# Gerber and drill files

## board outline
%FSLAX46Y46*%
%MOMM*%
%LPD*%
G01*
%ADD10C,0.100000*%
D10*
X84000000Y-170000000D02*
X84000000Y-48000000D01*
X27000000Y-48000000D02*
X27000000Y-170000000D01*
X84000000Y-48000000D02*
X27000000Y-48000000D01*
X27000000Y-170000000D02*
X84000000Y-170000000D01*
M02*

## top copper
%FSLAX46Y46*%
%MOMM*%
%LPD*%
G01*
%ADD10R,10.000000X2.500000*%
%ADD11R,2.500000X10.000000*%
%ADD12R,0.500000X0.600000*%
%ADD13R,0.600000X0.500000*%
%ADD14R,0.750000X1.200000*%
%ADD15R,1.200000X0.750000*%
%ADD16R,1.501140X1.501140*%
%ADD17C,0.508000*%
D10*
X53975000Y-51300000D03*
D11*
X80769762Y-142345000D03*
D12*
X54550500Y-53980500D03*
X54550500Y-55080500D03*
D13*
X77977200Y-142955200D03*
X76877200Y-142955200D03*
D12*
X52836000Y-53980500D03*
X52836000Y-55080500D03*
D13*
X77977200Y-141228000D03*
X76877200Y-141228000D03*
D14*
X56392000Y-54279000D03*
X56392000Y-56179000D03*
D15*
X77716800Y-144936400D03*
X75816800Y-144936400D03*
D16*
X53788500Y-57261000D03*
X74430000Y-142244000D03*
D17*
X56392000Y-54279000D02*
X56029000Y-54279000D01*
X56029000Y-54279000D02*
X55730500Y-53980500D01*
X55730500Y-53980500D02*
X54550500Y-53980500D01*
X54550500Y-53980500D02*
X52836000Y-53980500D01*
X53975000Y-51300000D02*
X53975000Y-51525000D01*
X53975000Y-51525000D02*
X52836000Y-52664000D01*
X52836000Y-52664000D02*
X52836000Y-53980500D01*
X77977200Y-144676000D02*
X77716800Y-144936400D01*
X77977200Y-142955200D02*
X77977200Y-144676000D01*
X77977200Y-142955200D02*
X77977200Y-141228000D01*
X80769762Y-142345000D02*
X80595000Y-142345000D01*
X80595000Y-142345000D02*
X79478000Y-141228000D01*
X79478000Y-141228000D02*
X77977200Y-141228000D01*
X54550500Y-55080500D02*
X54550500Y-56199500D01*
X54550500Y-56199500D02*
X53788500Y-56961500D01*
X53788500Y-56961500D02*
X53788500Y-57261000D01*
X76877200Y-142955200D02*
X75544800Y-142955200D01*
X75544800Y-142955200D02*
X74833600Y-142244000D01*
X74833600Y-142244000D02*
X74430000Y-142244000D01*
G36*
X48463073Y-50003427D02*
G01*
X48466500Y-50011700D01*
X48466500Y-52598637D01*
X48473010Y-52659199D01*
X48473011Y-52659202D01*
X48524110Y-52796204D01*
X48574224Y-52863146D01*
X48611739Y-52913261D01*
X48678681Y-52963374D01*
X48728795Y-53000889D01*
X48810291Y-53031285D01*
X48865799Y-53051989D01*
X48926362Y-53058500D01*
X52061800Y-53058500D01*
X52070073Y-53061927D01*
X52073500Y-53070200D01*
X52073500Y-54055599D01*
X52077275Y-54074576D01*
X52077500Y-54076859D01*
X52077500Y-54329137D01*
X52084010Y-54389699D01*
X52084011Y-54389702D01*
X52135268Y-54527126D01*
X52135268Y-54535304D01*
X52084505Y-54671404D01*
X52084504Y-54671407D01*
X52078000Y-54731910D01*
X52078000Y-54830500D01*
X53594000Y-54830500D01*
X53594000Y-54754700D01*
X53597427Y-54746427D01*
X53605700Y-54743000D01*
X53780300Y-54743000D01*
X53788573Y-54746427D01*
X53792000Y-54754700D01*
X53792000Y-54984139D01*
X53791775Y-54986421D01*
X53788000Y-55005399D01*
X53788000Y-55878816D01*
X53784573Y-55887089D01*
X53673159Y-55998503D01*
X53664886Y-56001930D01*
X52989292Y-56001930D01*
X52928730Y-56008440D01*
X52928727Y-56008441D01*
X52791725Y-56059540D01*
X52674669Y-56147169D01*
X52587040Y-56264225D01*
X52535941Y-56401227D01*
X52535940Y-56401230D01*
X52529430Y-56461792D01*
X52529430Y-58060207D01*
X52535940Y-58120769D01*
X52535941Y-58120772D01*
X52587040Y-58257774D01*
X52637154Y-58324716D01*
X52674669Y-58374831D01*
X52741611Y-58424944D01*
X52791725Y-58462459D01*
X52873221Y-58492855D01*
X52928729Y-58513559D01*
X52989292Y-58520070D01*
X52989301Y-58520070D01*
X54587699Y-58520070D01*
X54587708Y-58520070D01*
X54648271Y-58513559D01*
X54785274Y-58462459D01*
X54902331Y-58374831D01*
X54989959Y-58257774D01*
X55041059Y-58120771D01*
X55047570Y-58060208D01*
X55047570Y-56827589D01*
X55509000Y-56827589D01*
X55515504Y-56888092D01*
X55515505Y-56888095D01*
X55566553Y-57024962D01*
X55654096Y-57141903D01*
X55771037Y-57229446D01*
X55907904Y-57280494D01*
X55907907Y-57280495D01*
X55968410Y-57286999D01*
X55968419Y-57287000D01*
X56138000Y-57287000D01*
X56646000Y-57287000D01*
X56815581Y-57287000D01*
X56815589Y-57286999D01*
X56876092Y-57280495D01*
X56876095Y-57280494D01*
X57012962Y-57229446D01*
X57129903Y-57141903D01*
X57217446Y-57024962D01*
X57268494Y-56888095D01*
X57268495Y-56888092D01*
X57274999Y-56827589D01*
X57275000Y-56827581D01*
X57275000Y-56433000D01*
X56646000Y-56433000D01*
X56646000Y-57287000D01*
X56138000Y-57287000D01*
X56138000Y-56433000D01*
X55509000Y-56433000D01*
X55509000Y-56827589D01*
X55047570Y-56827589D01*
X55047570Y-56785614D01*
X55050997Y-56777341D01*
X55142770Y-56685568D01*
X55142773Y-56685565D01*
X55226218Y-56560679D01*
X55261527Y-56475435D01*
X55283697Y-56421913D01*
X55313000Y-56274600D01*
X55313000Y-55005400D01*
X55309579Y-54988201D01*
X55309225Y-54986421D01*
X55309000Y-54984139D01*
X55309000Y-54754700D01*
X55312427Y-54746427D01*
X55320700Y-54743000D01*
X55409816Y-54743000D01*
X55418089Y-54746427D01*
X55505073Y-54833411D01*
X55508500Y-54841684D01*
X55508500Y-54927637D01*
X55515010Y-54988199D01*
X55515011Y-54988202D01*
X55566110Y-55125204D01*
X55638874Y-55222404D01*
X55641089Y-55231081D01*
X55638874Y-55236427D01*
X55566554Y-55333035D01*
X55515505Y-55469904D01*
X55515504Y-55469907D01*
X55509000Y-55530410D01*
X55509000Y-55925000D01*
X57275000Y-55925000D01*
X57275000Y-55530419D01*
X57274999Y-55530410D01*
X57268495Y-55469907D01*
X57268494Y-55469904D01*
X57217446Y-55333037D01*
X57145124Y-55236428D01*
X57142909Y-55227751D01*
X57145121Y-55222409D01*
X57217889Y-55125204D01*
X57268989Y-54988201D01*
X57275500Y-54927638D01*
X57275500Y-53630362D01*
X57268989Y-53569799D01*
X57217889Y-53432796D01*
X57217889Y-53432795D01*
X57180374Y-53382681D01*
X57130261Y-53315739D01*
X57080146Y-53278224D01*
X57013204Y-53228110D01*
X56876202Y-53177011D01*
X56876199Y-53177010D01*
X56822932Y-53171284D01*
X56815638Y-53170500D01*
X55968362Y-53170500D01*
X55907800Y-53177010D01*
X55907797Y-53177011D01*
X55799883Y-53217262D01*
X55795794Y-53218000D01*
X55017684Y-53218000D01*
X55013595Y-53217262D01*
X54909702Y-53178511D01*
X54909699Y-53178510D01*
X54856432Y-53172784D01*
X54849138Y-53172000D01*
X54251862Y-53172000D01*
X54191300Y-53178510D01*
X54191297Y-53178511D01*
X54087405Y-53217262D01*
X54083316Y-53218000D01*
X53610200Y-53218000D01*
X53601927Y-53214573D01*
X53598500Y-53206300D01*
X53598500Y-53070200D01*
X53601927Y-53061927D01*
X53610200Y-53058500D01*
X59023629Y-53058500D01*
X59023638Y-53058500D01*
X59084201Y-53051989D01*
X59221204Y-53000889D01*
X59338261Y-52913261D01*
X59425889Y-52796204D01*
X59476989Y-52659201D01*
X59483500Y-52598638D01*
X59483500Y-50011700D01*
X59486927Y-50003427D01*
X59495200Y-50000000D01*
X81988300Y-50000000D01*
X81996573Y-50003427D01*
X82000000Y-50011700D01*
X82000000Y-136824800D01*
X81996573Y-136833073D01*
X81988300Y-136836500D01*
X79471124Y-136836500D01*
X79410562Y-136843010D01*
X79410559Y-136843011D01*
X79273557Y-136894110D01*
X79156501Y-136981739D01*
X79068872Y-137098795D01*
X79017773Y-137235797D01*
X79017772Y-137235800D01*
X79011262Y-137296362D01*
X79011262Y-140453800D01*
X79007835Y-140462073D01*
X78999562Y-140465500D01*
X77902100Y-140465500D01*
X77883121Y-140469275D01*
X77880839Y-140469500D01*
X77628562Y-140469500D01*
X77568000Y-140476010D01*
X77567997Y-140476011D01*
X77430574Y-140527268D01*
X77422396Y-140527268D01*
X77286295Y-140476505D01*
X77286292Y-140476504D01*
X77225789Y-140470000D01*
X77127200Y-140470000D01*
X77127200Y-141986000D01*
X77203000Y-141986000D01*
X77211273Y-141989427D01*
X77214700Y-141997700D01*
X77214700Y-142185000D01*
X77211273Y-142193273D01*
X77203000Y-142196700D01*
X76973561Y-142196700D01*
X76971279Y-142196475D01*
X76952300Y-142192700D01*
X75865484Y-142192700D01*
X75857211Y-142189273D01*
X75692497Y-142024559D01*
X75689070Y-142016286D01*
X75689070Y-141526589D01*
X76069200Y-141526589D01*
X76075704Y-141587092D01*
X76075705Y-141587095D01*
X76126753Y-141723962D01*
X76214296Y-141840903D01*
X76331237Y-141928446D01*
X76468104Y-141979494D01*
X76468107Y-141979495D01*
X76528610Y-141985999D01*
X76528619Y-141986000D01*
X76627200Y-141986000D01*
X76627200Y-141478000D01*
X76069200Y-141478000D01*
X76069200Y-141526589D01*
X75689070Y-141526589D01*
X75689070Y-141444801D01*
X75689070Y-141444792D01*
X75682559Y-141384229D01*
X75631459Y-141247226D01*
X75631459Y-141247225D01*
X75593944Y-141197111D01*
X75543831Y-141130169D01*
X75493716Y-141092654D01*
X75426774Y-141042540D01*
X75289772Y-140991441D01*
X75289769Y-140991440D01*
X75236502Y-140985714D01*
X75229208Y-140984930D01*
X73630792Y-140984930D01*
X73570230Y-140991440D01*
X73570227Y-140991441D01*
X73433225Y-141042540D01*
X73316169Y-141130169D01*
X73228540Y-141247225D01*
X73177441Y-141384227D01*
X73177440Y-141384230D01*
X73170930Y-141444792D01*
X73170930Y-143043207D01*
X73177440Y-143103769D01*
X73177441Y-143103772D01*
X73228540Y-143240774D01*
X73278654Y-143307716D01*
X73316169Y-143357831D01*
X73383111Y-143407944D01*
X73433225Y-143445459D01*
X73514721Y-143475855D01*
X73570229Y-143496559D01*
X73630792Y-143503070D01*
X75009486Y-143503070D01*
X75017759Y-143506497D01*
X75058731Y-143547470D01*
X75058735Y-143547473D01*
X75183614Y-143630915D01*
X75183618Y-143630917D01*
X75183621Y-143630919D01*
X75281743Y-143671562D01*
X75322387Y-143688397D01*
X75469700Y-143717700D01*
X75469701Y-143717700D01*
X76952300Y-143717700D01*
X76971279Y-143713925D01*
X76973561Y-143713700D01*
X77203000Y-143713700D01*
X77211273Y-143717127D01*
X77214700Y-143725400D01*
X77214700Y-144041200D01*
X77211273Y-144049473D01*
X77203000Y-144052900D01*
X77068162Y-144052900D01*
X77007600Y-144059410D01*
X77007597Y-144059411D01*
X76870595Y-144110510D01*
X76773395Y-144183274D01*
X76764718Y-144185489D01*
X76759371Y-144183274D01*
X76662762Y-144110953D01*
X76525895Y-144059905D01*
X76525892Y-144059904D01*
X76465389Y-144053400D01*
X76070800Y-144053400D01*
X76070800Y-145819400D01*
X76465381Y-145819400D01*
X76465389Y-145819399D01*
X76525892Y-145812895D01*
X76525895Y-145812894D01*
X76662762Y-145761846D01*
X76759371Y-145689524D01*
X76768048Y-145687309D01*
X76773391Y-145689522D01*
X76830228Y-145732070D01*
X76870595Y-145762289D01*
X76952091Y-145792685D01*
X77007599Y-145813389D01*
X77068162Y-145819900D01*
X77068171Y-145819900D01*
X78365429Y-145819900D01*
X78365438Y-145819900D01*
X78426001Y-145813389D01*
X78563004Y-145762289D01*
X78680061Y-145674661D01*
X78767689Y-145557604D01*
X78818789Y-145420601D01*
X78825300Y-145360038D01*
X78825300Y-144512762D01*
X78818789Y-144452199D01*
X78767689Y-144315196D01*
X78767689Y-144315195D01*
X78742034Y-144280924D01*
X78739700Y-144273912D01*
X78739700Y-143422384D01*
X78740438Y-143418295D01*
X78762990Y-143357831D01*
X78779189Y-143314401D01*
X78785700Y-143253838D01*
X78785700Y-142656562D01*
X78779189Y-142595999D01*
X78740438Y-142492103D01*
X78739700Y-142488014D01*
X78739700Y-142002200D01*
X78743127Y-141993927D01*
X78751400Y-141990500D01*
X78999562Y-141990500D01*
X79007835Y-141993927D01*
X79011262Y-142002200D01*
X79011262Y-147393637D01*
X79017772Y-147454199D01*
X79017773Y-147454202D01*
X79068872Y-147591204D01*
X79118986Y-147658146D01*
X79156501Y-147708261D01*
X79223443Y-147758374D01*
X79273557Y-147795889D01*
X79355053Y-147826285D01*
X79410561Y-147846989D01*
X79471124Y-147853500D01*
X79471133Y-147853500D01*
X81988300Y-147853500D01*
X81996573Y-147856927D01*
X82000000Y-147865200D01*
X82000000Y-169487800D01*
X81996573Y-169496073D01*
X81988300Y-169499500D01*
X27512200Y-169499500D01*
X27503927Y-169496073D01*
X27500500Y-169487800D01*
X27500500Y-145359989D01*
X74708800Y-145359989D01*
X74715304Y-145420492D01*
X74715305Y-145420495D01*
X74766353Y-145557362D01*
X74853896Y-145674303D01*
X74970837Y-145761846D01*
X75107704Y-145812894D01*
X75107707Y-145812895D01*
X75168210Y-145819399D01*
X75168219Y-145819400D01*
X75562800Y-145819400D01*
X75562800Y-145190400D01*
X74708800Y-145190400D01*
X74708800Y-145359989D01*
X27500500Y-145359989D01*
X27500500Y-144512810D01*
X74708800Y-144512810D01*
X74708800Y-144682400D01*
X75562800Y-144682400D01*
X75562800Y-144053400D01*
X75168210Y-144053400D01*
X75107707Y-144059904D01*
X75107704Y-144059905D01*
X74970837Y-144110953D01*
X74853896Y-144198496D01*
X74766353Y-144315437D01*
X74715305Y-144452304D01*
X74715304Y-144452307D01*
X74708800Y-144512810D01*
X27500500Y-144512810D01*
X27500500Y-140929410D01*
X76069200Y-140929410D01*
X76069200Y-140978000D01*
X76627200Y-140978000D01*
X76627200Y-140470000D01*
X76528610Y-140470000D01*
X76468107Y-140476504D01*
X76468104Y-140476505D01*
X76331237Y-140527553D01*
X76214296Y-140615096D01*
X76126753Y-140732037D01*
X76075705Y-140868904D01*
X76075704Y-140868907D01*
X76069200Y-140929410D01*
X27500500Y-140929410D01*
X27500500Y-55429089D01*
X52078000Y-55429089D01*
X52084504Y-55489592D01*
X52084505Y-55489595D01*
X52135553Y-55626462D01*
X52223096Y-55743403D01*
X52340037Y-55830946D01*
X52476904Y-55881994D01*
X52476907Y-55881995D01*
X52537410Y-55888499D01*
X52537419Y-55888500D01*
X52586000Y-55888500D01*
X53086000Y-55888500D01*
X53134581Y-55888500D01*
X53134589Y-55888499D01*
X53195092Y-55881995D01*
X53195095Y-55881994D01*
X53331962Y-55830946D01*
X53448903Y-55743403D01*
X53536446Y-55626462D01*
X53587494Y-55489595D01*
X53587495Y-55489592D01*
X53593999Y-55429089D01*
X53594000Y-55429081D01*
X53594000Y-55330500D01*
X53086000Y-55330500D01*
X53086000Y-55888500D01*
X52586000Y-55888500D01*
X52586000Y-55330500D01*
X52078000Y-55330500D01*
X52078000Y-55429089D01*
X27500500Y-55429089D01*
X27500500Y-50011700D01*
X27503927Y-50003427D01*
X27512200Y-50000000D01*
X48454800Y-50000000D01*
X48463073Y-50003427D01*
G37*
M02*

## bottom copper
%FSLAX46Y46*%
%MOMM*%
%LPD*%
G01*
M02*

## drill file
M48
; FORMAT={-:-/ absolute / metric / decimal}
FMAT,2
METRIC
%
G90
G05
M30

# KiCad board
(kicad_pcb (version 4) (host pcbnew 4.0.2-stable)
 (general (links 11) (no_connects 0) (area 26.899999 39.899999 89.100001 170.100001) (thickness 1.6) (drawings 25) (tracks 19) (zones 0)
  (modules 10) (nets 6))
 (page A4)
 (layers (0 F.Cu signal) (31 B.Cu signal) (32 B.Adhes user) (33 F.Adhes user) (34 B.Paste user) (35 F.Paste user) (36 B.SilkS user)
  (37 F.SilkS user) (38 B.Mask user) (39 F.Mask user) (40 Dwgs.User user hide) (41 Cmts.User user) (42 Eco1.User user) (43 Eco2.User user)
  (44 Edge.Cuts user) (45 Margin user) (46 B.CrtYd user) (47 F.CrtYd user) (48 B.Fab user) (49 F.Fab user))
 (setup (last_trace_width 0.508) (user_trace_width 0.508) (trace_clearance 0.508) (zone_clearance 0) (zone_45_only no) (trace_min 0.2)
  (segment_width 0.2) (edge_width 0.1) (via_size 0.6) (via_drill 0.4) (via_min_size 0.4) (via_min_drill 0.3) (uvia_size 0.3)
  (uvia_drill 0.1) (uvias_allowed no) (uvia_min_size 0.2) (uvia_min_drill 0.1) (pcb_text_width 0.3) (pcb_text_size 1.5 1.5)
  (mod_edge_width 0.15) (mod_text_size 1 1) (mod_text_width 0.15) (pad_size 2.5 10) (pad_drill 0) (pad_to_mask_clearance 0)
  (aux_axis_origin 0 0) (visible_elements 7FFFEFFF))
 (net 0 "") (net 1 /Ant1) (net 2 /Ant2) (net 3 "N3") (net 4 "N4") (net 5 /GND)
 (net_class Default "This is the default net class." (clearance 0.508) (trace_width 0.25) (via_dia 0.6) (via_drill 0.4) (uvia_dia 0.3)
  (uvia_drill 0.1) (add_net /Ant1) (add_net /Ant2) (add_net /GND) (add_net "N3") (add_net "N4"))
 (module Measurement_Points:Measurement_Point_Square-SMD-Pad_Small (layer F.Cu) (at 53.975 51.3)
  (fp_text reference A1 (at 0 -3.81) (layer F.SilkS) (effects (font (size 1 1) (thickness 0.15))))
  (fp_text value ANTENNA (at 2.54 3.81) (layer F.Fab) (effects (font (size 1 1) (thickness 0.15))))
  (pad 1 smd rect (at 0 0) (size 10 2.5) (layers F.Cu F.Mask) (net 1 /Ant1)))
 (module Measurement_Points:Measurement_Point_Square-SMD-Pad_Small (layer F.Cu) (at 80.769762 142.345)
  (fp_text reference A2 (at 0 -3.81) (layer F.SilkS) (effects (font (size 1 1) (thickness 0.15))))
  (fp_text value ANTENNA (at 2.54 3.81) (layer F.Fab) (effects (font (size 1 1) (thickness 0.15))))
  (pad 1 smd rect (at 0 0) (size 2.5 10) (layers F.Cu F.Mask) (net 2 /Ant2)))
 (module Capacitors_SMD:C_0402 (layer F.Cu) (at 54.5505 54.5305 270)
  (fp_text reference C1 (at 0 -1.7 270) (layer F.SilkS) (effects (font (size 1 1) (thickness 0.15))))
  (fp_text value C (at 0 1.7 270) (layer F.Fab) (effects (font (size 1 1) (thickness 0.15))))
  (pad 1 smd rect (at -0.55 0 270) (size 0.6 0.5) (layers F.Cu F.Paste F.Mask) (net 1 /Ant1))
  (pad 2 smd rect (at 0.55 0 270) (size 0.6 0.5) (layers F.Cu F.Paste F.Mask) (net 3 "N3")))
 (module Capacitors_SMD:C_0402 (layer F.Cu) (at 77.4272 142.9552 180)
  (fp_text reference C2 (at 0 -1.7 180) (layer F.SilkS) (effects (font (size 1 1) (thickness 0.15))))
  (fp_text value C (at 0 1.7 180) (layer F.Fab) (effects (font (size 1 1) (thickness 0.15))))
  (pad 1 smd rect (at -0.55 0 180) (size 0.6 0.5) (layers F.Cu F.Paste F.Mask) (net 2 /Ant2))
  (pad 2 smd rect (at 0.55 0 180) (size 0.6 0.5) (layers F.Cu F.Paste F.Mask) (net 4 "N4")))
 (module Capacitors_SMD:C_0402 (layer F.Cu) (at 52.836 54.5305 270)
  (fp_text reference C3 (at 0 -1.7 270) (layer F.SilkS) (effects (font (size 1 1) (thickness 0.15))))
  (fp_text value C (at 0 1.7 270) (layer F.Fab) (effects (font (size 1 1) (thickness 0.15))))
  (pad 1 smd rect (at -0.55 0 270) (size 0.6 0.5) (layers F.Cu F.Paste F.Mask) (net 1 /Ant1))
  (pad 2 smd rect (at 0.55 0 270) (size 0.6 0.5) (layers F.Cu F.Paste F.Mask) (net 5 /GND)))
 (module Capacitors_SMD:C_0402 (layer F.Cu) (at 77.4272 141.228 180)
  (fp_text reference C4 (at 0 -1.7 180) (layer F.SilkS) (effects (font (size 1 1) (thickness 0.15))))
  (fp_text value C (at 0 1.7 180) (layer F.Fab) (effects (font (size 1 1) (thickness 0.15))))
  (pad 1 smd rect (at -0.55 0 180) (size 0.6 0.5) (layers F.Cu F.Paste F.Mask) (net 2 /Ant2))
  (pad 2 smd rect (at 0.55 0 180) (size 0.6 0.5) (layers F.Cu F.Paste F.Mask) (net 5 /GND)))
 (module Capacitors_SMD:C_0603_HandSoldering (layer F.Cu) (at 56.392 55.229 270)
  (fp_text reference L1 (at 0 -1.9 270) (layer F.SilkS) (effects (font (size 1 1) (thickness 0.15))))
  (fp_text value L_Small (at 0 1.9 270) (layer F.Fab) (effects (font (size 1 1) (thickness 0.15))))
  (pad 1 smd rect (at -0.95 0 270) (size 1.2 0.75) (layers F.Cu F.Paste F.Mask) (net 1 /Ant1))
  (pad 2 smd rect (at 0.95 0 270) (size 1.2 0.75) (layers F.Cu F.Paste F.Mask) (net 5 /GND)))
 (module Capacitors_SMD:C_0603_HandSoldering (layer F.Cu) (at 76.7668 144.9364 180)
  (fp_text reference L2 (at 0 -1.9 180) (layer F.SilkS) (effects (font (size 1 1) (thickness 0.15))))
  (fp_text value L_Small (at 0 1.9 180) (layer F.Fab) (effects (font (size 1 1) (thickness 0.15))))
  (pad 1 smd rect (at -0.95 0 180) (size 1.2 0.75) (layers F.Cu F.Paste F.Mask) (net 2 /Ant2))
  (pad 2 smd rect (at 0.95 0 180) (size 1.2 0.75) (layers F.Cu F.Paste F.Mask) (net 5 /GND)))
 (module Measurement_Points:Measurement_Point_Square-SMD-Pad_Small (layer F.Cu) (at 53.7885 57.261)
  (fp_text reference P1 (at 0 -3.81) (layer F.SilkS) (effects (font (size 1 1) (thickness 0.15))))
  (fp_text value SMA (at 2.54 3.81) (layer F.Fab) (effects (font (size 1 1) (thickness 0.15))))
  (pad 1 smd rect (at 0 0) (size 1.50114 1.50114) (layers F.Cu F.Mask) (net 3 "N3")))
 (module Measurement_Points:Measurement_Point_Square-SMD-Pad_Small (layer F.Cu) (at 74.43 142.244)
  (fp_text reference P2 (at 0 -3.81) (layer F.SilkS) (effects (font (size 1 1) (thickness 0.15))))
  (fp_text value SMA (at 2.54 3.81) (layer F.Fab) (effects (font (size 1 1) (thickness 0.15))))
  (pad 1 smd rect (at 0 0) (size 1.50114 1.50114) (layers F.Cu F.Mask) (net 4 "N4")))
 (gr_line (start 84 170) (end 84 48) (angle 90) (layer Edge.Cuts) (width 0.1))
 (gr_line (start 27 48) (end 27 170) (angle 90) (layer Edge.Cuts) (width 0.1))
 (gr_line (start 84 48) (end 27 48) (angle 90) (layer Edge.Cuts) (width 0.1))
 (gr_line (start 27 170) (end 84 170) (angle 90) (layer Edge.Cuts) (width 0.1))
 (segment (start 56.392 54.279) (end 56.029 54.279) (width 0.508) (layer F.Cu) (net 1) (status C00000))
 (segment (start 56.029 54.279) (end 55.7305 53.9805) (width 0.508) (layer F.Cu) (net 1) (status 400000))
 (segment (start 55.7305 53.9805) (end 54.5505 53.9805) (width 0.508) (layer F.Cu) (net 1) (status 800000))
 (segment (start 54.5505 53.9805) (end 52.836 53.9805) (width 0.508) (layer F.Cu) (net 1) (status C00000))
 (segment (start 53.975 51.3) (end 53.975 51.525) (width 0.508) (layer F.Cu) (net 1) (status C00000))
 (segment (start 53.975 51.525) (end 52.836 52.664) (width 0.508) (layer F.Cu) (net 1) (status 400000))
 (segment (start 52.836 52.664) (end 52.836 53.9805) (width 0.508) (layer F.Cu) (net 1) (status 800000))
 (segment (start 77.9772 144.676) (end 77.7168 144.9364) (width 0.508) (layer F.Cu) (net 2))
 (segment (start 77.9772 142.9552) (end 77.9772 144.676) (width 0.508) (layer F.Cu) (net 2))
 (segment (start 77.9772 142.9552) (end 77.9772 141.228) (width 0.508) (layer F.Cu) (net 2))
 (segment (start 80.769762 142.345) (end 80.595 142.345) (width 0.508) (layer F.Cu) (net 2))
 (segment (start 80.595 142.345) (end 79.478 141.228) (width 0.508) (layer F.Cu) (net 2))
 (segment (start 79.478 141.228) (end 77.9772 141.228) (width 0.508) (layer F.Cu) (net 2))
 (segment (start 54.5505 55.0805) (end 54.5505 56.1995) (width 0.508) (layer F.Cu) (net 3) (status 400000))
 (segment (start 54.5505 56.1995) (end 53.7885 56.9615) (width 0.508) (layer F.Cu) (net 3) (status 800000))
 (segment (start 53.7885 56.9615) (end 53.7885 57.261) (width 0.508) (layer F.Cu) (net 3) (status C00000))
 (segment (start 76.8772 142.9552) (end 75.5448 142.9552) (width 0.508) (layer F.Cu) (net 4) (status 400000))
 (segment (start 75.5448 142.9552) (end 74.8336 142.244) (width 0.508) (layer F.Cu) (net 4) (status 800000))
 (segment (start 74.8336 142.244) (end 74.43 142.244) (width 0.508) (layer F.Cu) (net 4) (status C00000))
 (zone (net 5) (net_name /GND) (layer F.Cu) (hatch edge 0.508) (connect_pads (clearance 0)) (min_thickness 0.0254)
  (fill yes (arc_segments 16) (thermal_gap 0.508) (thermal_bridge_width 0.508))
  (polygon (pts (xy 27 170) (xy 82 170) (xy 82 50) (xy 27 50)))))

